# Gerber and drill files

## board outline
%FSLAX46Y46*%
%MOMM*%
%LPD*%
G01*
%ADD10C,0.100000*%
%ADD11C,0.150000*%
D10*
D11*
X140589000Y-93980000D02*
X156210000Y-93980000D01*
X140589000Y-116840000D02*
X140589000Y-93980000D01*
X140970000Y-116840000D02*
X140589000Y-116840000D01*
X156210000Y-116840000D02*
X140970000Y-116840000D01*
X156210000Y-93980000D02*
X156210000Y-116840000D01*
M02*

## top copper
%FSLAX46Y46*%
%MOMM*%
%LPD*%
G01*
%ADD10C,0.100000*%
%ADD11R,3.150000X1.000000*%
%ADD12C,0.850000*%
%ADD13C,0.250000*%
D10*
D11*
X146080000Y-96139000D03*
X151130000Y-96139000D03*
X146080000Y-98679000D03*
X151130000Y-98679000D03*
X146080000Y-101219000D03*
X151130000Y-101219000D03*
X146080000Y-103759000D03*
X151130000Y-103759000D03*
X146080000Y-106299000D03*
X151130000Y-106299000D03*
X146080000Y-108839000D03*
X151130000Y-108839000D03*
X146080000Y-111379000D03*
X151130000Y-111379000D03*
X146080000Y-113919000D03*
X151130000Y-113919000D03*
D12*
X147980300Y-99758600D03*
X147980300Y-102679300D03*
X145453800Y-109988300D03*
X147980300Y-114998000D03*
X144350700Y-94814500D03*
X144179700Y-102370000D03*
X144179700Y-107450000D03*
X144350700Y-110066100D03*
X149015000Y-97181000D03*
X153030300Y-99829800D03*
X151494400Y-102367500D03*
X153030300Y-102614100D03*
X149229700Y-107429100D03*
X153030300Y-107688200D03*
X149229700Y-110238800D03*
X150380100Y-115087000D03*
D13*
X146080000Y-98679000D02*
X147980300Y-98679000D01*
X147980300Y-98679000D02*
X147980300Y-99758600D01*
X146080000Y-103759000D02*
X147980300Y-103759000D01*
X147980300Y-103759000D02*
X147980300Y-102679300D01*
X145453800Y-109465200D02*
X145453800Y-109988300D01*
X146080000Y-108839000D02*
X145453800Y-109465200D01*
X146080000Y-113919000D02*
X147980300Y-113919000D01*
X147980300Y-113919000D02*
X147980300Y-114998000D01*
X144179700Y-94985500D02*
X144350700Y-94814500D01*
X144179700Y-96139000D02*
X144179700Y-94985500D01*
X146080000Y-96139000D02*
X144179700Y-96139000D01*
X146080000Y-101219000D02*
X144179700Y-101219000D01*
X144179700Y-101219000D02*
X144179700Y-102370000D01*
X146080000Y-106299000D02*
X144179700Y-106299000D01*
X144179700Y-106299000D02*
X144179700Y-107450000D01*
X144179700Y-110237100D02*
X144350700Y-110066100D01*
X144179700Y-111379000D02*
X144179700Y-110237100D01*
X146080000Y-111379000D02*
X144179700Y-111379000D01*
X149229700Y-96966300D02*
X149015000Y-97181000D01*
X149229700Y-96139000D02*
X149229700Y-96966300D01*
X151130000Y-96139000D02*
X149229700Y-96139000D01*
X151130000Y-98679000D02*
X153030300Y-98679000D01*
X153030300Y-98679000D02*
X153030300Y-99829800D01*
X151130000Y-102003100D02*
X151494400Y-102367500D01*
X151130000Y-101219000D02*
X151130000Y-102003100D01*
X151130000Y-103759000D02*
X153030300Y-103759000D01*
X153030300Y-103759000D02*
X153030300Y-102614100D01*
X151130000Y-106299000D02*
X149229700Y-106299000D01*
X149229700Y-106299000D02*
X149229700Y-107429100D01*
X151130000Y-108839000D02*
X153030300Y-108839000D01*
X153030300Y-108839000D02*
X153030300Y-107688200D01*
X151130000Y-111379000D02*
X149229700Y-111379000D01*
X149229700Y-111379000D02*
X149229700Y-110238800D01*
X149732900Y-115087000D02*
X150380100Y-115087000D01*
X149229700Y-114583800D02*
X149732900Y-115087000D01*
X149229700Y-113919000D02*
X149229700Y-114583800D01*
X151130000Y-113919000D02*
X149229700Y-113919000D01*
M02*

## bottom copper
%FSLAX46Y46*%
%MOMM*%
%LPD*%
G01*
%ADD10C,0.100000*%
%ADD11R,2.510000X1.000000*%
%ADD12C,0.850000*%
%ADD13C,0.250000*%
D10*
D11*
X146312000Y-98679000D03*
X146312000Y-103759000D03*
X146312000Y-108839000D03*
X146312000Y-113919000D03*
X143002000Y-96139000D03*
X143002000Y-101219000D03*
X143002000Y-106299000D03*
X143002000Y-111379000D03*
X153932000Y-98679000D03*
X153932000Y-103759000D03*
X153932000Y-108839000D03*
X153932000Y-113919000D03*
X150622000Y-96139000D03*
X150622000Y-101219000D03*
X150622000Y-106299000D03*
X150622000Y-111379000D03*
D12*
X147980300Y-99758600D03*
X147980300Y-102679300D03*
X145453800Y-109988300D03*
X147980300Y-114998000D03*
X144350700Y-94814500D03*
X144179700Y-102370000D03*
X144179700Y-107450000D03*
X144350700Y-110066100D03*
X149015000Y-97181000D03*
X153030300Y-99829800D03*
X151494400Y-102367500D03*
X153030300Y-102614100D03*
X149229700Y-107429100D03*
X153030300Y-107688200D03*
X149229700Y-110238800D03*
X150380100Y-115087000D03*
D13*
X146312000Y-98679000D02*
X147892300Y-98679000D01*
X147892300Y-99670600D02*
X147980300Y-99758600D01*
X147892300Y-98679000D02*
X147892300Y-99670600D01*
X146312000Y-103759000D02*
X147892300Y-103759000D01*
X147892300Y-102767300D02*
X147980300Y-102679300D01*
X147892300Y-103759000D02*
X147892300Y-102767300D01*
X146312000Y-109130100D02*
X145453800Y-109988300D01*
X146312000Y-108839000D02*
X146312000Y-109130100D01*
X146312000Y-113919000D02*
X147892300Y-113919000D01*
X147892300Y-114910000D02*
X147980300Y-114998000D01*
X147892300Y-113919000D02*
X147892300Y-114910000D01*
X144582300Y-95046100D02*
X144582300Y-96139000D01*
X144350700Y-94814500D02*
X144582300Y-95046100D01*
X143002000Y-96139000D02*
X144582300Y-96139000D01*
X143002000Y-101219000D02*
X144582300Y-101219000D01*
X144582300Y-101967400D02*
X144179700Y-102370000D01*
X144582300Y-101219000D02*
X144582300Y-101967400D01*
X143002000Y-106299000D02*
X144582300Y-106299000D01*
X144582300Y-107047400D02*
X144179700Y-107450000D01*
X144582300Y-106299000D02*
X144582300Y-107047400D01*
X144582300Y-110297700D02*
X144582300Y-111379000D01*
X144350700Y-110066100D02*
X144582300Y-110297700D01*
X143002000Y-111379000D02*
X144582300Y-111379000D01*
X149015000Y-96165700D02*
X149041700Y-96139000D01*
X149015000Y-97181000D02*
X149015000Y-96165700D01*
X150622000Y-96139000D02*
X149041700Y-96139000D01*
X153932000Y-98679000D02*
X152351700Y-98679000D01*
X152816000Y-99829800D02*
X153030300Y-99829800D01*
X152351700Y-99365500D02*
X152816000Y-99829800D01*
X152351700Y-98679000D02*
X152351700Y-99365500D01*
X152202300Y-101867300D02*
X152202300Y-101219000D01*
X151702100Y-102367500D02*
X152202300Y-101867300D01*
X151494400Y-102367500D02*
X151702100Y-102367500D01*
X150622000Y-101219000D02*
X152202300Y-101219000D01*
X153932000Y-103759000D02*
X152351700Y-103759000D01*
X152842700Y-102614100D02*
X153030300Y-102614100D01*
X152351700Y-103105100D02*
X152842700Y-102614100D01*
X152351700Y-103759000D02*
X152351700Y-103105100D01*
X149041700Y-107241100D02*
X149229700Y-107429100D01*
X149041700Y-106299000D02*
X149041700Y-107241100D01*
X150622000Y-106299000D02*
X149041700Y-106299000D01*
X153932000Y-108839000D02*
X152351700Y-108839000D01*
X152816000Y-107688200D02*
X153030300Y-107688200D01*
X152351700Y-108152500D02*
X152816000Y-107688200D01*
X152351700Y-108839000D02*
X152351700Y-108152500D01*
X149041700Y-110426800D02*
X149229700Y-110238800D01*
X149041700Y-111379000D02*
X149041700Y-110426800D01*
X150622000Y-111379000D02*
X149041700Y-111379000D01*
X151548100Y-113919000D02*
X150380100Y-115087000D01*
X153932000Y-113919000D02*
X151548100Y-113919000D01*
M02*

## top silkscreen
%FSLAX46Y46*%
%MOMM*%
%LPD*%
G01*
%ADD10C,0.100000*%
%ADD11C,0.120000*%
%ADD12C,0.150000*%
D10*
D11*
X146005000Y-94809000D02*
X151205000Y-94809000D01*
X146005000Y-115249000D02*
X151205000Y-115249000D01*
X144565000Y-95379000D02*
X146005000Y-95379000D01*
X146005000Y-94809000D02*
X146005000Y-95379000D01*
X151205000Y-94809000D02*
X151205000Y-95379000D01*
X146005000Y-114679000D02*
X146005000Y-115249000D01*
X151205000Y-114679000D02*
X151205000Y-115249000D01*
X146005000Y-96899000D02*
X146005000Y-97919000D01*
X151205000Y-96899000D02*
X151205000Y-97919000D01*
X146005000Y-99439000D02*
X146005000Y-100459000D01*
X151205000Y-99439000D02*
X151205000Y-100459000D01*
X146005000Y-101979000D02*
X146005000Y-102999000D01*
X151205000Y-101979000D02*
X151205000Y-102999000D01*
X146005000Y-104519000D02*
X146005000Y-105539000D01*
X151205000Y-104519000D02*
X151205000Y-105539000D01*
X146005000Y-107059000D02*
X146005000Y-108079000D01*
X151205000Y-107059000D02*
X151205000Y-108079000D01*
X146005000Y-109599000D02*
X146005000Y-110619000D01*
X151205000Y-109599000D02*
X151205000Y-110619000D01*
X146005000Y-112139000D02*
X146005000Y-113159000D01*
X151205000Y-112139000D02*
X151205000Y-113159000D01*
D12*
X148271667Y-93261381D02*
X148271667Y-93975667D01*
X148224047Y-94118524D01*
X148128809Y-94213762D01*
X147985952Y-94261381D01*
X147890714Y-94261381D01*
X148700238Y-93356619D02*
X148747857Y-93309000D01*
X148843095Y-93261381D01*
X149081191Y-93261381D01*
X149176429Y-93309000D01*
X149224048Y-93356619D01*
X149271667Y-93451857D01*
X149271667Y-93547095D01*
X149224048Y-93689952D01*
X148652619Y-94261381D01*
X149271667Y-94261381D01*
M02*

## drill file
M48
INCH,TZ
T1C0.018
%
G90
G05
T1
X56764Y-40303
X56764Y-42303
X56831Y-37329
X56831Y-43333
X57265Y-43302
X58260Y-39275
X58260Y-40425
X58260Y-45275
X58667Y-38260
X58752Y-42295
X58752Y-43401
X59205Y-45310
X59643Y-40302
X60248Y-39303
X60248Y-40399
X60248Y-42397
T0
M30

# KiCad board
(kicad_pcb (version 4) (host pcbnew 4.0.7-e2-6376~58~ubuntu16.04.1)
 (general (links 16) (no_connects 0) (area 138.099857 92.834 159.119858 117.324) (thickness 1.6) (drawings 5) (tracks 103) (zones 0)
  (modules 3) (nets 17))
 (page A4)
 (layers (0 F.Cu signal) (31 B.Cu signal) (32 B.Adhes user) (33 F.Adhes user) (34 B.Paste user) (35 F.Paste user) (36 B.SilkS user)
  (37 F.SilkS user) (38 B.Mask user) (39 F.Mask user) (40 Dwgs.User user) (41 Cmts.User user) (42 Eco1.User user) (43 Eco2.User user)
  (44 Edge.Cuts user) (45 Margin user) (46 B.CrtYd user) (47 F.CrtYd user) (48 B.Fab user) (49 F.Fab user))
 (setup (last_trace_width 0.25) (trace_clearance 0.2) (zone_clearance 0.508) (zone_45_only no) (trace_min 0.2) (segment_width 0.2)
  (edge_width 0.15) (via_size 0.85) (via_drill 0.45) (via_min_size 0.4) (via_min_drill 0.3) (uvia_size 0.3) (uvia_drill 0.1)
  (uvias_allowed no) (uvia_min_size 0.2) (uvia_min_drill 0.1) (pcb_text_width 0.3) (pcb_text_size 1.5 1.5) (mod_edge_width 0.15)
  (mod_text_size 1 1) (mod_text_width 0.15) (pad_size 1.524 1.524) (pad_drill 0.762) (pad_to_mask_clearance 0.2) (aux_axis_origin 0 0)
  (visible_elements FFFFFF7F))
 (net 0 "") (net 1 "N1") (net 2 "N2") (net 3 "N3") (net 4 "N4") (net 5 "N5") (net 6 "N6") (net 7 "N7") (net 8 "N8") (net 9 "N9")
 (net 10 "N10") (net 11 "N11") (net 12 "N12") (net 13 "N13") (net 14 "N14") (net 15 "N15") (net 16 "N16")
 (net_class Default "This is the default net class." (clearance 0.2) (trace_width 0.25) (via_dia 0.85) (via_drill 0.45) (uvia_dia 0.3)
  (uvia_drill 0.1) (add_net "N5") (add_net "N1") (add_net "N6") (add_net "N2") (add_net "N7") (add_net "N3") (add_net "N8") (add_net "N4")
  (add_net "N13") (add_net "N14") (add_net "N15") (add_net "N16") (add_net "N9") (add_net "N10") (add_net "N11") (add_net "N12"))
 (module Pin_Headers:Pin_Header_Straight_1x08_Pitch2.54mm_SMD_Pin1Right (layer B.Cu) (at 144.657 105.029 180)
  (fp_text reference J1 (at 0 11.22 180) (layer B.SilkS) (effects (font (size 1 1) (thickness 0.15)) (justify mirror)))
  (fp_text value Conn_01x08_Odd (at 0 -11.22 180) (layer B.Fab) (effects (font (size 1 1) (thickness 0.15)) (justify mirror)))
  (pad 2 smd rect (at -1.655 6.35 180) (size 2.51 1) (layers B.Cu B.Paste B.Mask) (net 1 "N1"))
  (pad 4 smd rect (at -1.655 1.27 180) (size 2.51 1) (layers B.Cu B.Paste B.Mask) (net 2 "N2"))
  (pad 6 smd rect (at -1.655 -3.81 180) (size 2.51 1) (layers B.Cu B.Paste B.Mask) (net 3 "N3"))
  (pad 8 smd rect (at -1.655 -8.89 180) (size 2.51 1) (layers B.Cu B.Paste B.Mask) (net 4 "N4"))
  (pad 1 smd rect (at 1.655 8.89 180) (size 2.51 1) (layers B.Cu B.Paste B.Mask) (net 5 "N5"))
  (pad 3 smd rect (at 1.655 3.81 180) (size 2.51 1) (layers B.Cu B.Paste B.Mask) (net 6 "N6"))
  (pad 5 smd rect (at 1.655 -1.27 180) (size 2.51 1) (layers B.Cu B.Paste B.Mask) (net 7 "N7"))
  (pad 7 smd rect (at 1.655 -6.35 180) (size 2.51 1) (layers B.Cu B.Paste B.Mask) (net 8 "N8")))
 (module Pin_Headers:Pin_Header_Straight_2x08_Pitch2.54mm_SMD (layer F.Cu) (at 148.605 105.029)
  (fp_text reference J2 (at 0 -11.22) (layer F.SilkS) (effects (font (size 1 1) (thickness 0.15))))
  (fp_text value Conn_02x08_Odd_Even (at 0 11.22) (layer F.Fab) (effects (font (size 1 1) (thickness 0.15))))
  (fp_line (start -2.6 -10.22) (end 2.6 -10.22) (layer F.SilkS) (width 0.12))
  (fp_line (start -2.6 10.22) (end 2.6 10.22) (layer F.SilkS) (width 0.12))
  (fp_line (start -4.04 -9.65) (end -2.6 -9.65) (layer F.SilkS) (width 0.12))
  (fp_line (start -2.6 -10.22) (end -2.6 -9.65) (layer F.SilkS) (width 0.12))
  (fp_line (start 2.6 -10.22) (end 2.6 -9.65) (layer F.SilkS) (width 0.12))
  (fp_line (start -2.6 9.65) (end -2.6 10.22) (layer F.SilkS) (width 0.12))
  (fp_line (start 2.6 9.65) (end 2.6 10.22) (layer F.SilkS) (width 0.12))
  (fp_line (start -2.6 -8.13) (end -2.6 -7.11) (layer F.SilkS) (width 0.12))
  (fp_line (start 2.6 -8.13) (end 2.6 -7.11) (layer F.SilkS) (width 0.12))
  (fp_line (start -2.6 -5.59) (end -2.6 -4.57) (layer F.SilkS) (width 0.12))
  (fp_line (start 2.6 -5.59) (end 2.6 -4.57) (layer F.SilkS) (width 0.12))
  (fp_line (start -2.6 -3.05) (end -2.6 -2.03) (layer F.SilkS) (width 0.12))
  (fp_line (start 2.6 -3.05) (end 2.6 -2.03) (layer F.SilkS) (width 0.12))
  (fp_line (start -2.6 -0.51) (end -2.6 0.51) (layer F.SilkS) (width 0.12))
  (fp_line (start 2.6 -0.51) (end 2.6 0.51) (layer F.SilkS) (width 0.12))
  (fp_line (start -2.6 2.03) (end -2.6 3.05) (layer F.SilkS) (width 0.12))
  (fp_line (start 2.6 2.03) (end 2.6 3.05) (layer F.SilkS) (width 0.12))
  (fp_line (start -2.6 4.57) (end -2.6 5.59) (layer F.SilkS) (width 0.12))
  (fp_line (start 2.6 4.57) (end 2.6 5.59) (layer F.SilkS) (width 0.12))
  (fp_line (start -2.6 7.11) (end -2.6 8.13) (layer F.SilkS) (width 0.12))
  (fp_line (start 2.6 7.11) (end 2.6 8.13) (layer F.SilkS) (width 0.12))
  (pad 1 smd rect (at -2.525 -8.89) (size 3.15 1) (layers F.Cu F.Paste F.Mask) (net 5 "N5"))
  (pad 2 smd rect (at 2.525 -8.89) (size 3.15 1) (layers F.Cu F.Paste F.Mask) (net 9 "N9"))
  (pad 3 smd rect (at -2.525 -6.35) (size 3.15 1) (layers F.Cu F.Paste F.Mask) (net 1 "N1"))
  (pad 4 smd rect (at 2.525 -6.35) (size 3.15 1) (layers F.Cu F.Paste F.Mask) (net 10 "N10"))
  (pad 5 smd rect (at -2.525 -3.81) (size 3.15 1) (layers F.Cu F.Paste F.Mask) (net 6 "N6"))
  (pad 6 smd rect (at 2.525 -3.81) (size 3.15 1) (layers F.Cu F.Paste F.Mask) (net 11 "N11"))
  (pad 7 smd rect (at -2.525 -1.27) (size 3.15 1) (layers F.Cu F.Paste F.Mask) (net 2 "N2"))
  (pad 8 smd rect (at 2.525 -1.27) (size 3.15 1) (layers F.Cu F.Paste F.Mask) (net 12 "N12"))
  (pad 9 smd rect (at -2.525 1.27) (size 3.15 1) (layers F.Cu F.Paste F.Mask) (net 7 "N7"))
  (pad 10 smd rect (at 2.525 1.27) (size 3.15 1) (layers F.Cu F.Paste F.Mask) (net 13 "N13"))
  (pad 11 smd rect (at -2.525 3.81) (size 3.15 1) (layers F.Cu F.Paste F.Mask) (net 3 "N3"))
  (pad 12 smd rect (at 2.525 3.81) (size 3.15 1) (layers F.Cu F.Paste F.Mask) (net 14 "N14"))
  (pad 13 smd rect (at -2.525 6.35) (size 3.15 1) (layers F.Cu F.Paste F.Mask) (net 8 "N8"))
  (pad 14 smd rect (at 2.525 6.35) (size 3.15 1) (layers F.Cu F.Paste F.Mask) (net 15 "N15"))
  (pad 15 smd rect (at -2.525 8.89) (size 3.15 1) (layers F.Cu F.Paste F.Mask) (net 4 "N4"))
  (pad 16 smd rect (at 2.525 8.89) (size 3.15 1) (layers F.Cu F.Paste F.Mask) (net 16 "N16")))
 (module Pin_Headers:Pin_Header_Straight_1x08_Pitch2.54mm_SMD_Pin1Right (layer B.Cu) (at 152.277 105.029 180)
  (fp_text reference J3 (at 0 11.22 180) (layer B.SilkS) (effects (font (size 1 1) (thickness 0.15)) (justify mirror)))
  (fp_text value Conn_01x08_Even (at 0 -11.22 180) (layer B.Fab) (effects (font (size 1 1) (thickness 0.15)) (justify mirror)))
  (pad 2 smd rect (at -1.655 6.35 180) (size 2.51 1) (layers B.Cu B.Paste B.Mask) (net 10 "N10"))
  (pad 4 smd rect (at -1.655 1.27 180) (size 2.51 1) (layers B.Cu B.Paste B.Mask) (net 12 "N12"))
  (pad 6 smd rect (at -1.655 -3.81 180) (size 2.51 1) (layers B.Cu B.Paste B.Mask) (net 14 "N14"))
  (pad 8 smd rect (at -1.655 -8.89 180) (size 2.51 1) (layers B.Cu B.Paste B.Mask) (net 16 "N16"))
  (pad 1 smd rect (at 1.655 8.89 180) (size 2.51 1) (layers B.Cu B.Paste B.Mask) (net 9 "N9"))
  (pad 3 smd rect (at 1.655 3.81 180) (size 2.51 1) (layers B.Cu B.Paste B.Mask) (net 11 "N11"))
  (pad 5 smd rect (at 1.655 -1.27 180) (size 2.51 1) (layers B.Cu B.Paste B.Mask) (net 13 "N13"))
  (pad 7 smd rect (at 1.655 -6.35 180) (size 2.51 1) (layers B.Cu B.Paste B.Mask) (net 15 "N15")))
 (gr_line (start 140.589 93.98) (end 156.21 93.98) (layer Edge.Cuts) (width 0.15))
 (gr_line (start 140.589 116.84) (end 140.589 93.98) (layer Edge.Cuts) (width 0.15))
 (gr_line (start 140.97 116.84) (end 140.589 116.84) (layer Edge.Cuts) (width 0.15))
 (gr_line (start 156.21 116.84) (end 140.97 116.84) (layer Edge.Cuts) (width 0.15))
 (gr_line (start 156.21 93.98) (end 156.21 116.84) (layer Edge.Cuts) (width 0.15))
 (via (at 147.9803 99.7586) (size 0.85) (layers F.Cu B.Cu) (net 1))
 (segment (start 146.08 98.679) (end 147.9803 98.679) (width 0.25) (layer F.Cu) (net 1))
 (segment (start 146.312 98.679) (end 147.8923 98.679) (width 0.25) (layer B.Cu) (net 1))
 (segment (start 147.8923 99.6706) (end 147.9803 99.7586) (width 0.25) (layer B.Cu) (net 1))
 (segment (start 147.8923 98.679) (end 147.8923 99.6706) (width 0.25) (layer B.Cu) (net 1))
 (segment (start 147.9803 98.679) (end 147.9803 99.7586) (width 0.25) (layer F.Cu) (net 1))
 (via (at 147.9803 102.6793) (size 0.85) (layers F.Cu B.Cu) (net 2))
 (segment (start 146.08 103.759) (end 147.9803 103.759) (width 0.25) (layer F.Cu) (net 2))
 (segment (start 146.312 103.759) (end 147.8923 103.759) (width 0.25) (layer B.Cu) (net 2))
 (segment (start 147.8923 102.7673) (end 147.9803 102.6793) (width 0.25) (layer B.Cu) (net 2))
 (segment (start 147.8923 103.759) (end 147.8923 102.7673) (width 0.25) (layer B.Cu) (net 2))
 (segment (start 147.9803 103.759) (end 147.9803 102.6793) (width 0.25) (layer F.Cu) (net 2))
 (via (at 145.4538 109.9883) (size 0.85) (layers F.Cu B.Cu) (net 3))
 (segment (start 146.312 109.1301) (end 145.4538 109.9883) (width 0.25) (layer B.Cu) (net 3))
 (segment (start 146.312 108.839) (end 146.312 109.1301) (width 0.25) (layer B.Cu) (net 3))
 (segment (start 145.4538 109.4652) (end 145.4538 109.9883) (width 0.25) (layer F.Cu) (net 3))
 (segment (start 146.08 108.839) (end 145.4538 109.4652) (width 0.25) (layer F.Cu) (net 3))
 (via (at 147.9803 114.998) (size 0.85) (layers F.Cu B.Cu) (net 4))
 (segment (start 146.08 113.919) (end 147.9803 113.919) (width 0.25) (layer F.Cu) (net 4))
 (segment (start 146.312 113.919) (end 147.8923 113.919) (width 0.25) (layer B.Cu) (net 4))
 (segment (start 147.8923 114.91) (end 147.9803 114.998) (width 0.25) (layer B.Cu) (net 4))
 (segment (start 147.8923 113.919) (end 147.8923 114.91) (width 0.25) (layer B.Cu) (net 4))
 (segment (start 147.9803 113.919) (end 147.9803 114.998) (width 0.25) (layer F.Cu) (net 4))
 (via (at 144.3507 94.8145) (size 0.85) (layers F.Cu B.Cu) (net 5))
 (segment (start 144.1797 94.9855) (end 144.3507 94.8145) (width 0.25) (layer F.Cu) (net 5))
 (segment (start 144.1797 96.139) (end 144.1797 94.9855) (width 0.25) (layer F.Cu) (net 5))
 (segment (start 144.5823 95.0461) (end 144.5823 96.139) (width 0.25) (layer B.Cu) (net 5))
 (segment (start 144.3507 94.8145) (end 144.5823 95.0461) (width 0.25) (layer B.Cu) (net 5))
 (segment (start 146.08 96.139) (end 144.1797 96.139) (width 0.25) (layer F.Cu) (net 5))
 (segment (start 143.002 96.139) (end 144.5823 96.139) (width 0.25) (layer B.Cu) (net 5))
 (via (at 144.1797 102.37) (size 0.85) (layers F.Cu B.Cu) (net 6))
 (segment (start 146.08 101.219) (end 144.1797 101.219) (width 0.25) (layer F.Cu) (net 6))
 (segment (start 143.002 101.219) (end 144.5823 101.219) (width 0.25) (layer B.Cu) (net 6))
 (segment (start 144.5823 101.9674) (end 144.1797 102.37) (width 0.25) (layer B.Cu) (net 6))
 (segment (start 144.5823 101.219) (end 144.5823 101.9674) (width 0.25) (layer B.Cu) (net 6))
 (segment (start 144.1797 101.219) (end 144.1797 102.37) (width 0.25) (layer F.Cu) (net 6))
 (via (at 144.1797 107.45) (size 0.85) (layers F.Cu B.Cu) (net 7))
 (segment (start 146.08 106.299) (end 144.1797 106.299) (width 0.25) (layer F.Cu) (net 7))
 (segment (start 143.002 106.299) (end 144.5823 106.299) (width 0.25) (layer B.Cu) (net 7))
 (segment (start 144.5823 107.0474) (end 144.1797 107.45) (width 0.25) (layer B.Cu) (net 7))
 (segment (start 144.5823 106.299) (end 144.5823 107.0474) (width 0.25) (layer B.Cu) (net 7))
 (segment (start 144.1797 106.299) (end 144.1797 107.45) (width 0.25) (layer F.Cu) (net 7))
 (via (at 144.3507 110.0661) (size 0.85) (layers F.Cu B.Cu) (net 8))
 (segment (start 144.1797 110.2371) (end 144.3507 110.0661) (width 0.25) (layer F.Cu) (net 8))
 (segment (start 144.1797 111.379) (end 144.1797 110.2371) (width 0.25) (layer F.Cu) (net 8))
 (segment (start 144.5823 110.2977) (end 144.5823 111.379) (width 0.25) (layer B.Cu) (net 8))
 (segment (start 144.3507 110.0661) (end 144.5823 110.2977) (width 0.25) (layer B.Cu) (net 8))
 (segment (start 146.08 111.379) (end 144.1797 111.379) (width 0.25) (layer F.Cu) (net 8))
 (segment (start 143.002 111.379) (end 144.5823 111.379) (width 0.25) (layer B.Cu) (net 8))
 (via (at 149.015 97.181) (size 0.85) (layers F.Cu B.Cu) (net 9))
 (segment (start 149.015 96.1657) (end 149.0417 96.139) (width 0.25) (layer B.Cu) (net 9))
 (segment (start 149.015 97.181) (end 149.015 96.1657) (width 0.25) (layer B.Cu) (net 9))
 (segment (start 149.2297 96.9663) (end 149.015 97.181) (width 0.25) (layer F.Cu) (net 9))
 (segment (start 149.2297 96.139) (end 149.2297 96.9663) (width 0.25) (layer F.Cu) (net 9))
 (segment (start 150.622 96.139) (end 149.0417 96.139) (width 0.25) (layer B.Cu) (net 9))
 (segment (start 151.13 96.139) (end 149.2297 96.139) (width 0.25) (layer F.Cu) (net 9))
 (via (at 153.0303 99.8298) (size 0.85) (layers F.Cu B.Cu) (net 10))
 (segment (start 151.13 98.679) (end 153.0303 98.679) (width 0.25) (layer F.Cu) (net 10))
 (segment (start 153.932 98.679) (end 152.3517 98.679) (width 0.25) (layer B.Cu) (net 10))
 (segment (start 152.816 99.8298) (end 153.0303 99.8298) (width 0.25) (layer B.Cu) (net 10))
 (segment (start 152.3517 99.3655) (end 152.816 99.8298) (width 0.25) (layer B.Cu) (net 10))
 (segment (start 152.3517 98.679) (end 152.3517 99.3655) (width 0.25) (layer B.Cu) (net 10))
 (segment (start 153.0303 98.679) (end 153.0303 99.8298) (width 0.25) (layer F.Cu) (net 10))
 (via (at 151.4944 102.3675) (size 0.85) (layers F.Cu B.Cu) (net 11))
 (segment (start 152.2023 101.8673) (end 152.2023 101.219) (width 0.25) (layer B.Cu) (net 11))
 (segment (start 151.7021 102.3675) (end 152.2023 101.8673) (width 0.25) (layer B.Cu) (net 11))
 (segment (start 151.4944 102.3675) (end 151.7021 102.3675) (width 0.25) (layer B.Cu) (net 11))
 (segment (start 151.13 102.0031) (end 151.4944 102.3675) (width 0.25) (layer F.Cu) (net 11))
 (segment (start 151.13 101.219) (end 151.13 102.0031) (width 0.25) (layer F.Cu) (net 11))
 (segment (start 150.622 101.219) (end 152.2023 101.219) (width 0.25) (layer B.Cu) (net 11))
 (via (at 153.0303 102.6141) (size 0.85) (layers F.Cu B.Cu) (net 12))
 (segment (start 151.13 103.759) (end 153.0303 103.759) (width 0.25) (layer F.Cu) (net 12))
 (segment (start 153.932 103.759) (end 152.3517 103.759) (width 0.25) (layer B.Cu) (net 12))
 (segment (start 152.8427 102.6141) (end 153.0303 102.6141) (width 0.25) (layer B.Cu) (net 12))
 (segment (start 152.3517 103.1051) (end 152.8427 102.6141) (width 0.25) (layer B.Cu) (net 12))
 (segment (start 152.3517 103.759) (end 152.3517 103.1051) (width 0.25) (layer B.Cu) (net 12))
 (segment (start 153.0303 103.759) (end 153.0303 102.6141) (width 0.25) (layer F.Cu) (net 12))
 (via (at 149.2297 107.4291) (size 0.85) (layers F.Cu B.Cu) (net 13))
 (segment (start 151.13 106.299) (end 149.2297 106.299) (width 0.25) (layer F.Cu) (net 13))
 (segment (start 149.0417 107.2411) (end 149.2297 107.4291) (width 0.25) (layer B.Cu) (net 13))
 (segment (start 149.0417 106.299) (end 149.0417 107.2411) (width 0.25) (layer B.Cu) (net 13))
 (segment (start 149.2297 106.299) (end 149.2297 107.4291) (width 0.25) (layer F.Cu) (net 13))
 (segment (start 150.622 106.299) (end 149.0417 106.299) (width 0.25) (layer B.Cu) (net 13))
 (via (at 153.0303 107.6882) (size 0.85) (layers F.Cu B.Cu) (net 14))
 (segment (start 151.13 108.839) (end 153.0303 108.839) (width 0.25) (layer F.Cu) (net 14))
 (segment (start 153.932 108.839) (end 152.3517 108.839) (width 0.25) (layer B.Cu) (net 14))
 (segment (start 152.816 107.6882) (end 153.0303 107.6882) (width 0.25) (layer B.Cu) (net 14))
 (segment (start 152.3517 108.1525) (end 152.816 107.6882) (width 0.25) (layer B.Cu) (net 14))
 (segment (start 152.3517 108.839) (end 152.3517 108.1525) (width 0.25) (layer B.Cu) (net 14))
 (segment (start 153.0303 108.839) (end 153.0303 107.6882) (width 0.25) (layer F.Cu) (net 14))
 (via (at 149.2297 110.2388) (size 0.85) (layers F.Cu B.Cu) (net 15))
 (segment (start 151.13 111.379) (end 149.2297 111.379) (width 0.25) (layer F.Cu) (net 15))
 (segment (start 149.0417 110.4268) (end 149.2297 110.2388) (width 0.25) (layer B.Cu) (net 15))
 (segment (start 149.0417 111.379) (end 149.0417 110.4268) (width 0.25) (layer B.Cu) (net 15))
 (segment (start 149.2297 111.379) (end 149.2297 110.2388) (width 0.25) (layer F.Cu) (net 15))
 (segment (start 150.622 111.379) (end 149.0417 111.379) (width 0.25) (layer B.Cu) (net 15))
 (via (at 150.3801 115.087) (size 0.85) (layers F.Cu B.Cu) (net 16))
 (segment (start 151.5481 113.919) (end 150.3801 115.087) (width 0.25) (layer B.Cu) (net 16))
 (segment (start 153.932 113.919) (end 151.5481 113.919) (width 0.25) (layer B.Cu) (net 16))
 (segment (start 149.7329 115.087) (end 150.3801 115.087) (width 0.25) (layer F.Cu) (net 16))
 (segment (start 149.2297 114.5838) (end 149.7329 115.087) (width 0.25) (layer F.Cu) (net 16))
 (segment (start 149.2297 113.919) (end 149.2297 114.5838) (width 0.25) (layer F.Cu) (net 16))
 (segment (start 151.13 113.919) (end 149.2297 113.919) (width 0.25) (layer F.Cu) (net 16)))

